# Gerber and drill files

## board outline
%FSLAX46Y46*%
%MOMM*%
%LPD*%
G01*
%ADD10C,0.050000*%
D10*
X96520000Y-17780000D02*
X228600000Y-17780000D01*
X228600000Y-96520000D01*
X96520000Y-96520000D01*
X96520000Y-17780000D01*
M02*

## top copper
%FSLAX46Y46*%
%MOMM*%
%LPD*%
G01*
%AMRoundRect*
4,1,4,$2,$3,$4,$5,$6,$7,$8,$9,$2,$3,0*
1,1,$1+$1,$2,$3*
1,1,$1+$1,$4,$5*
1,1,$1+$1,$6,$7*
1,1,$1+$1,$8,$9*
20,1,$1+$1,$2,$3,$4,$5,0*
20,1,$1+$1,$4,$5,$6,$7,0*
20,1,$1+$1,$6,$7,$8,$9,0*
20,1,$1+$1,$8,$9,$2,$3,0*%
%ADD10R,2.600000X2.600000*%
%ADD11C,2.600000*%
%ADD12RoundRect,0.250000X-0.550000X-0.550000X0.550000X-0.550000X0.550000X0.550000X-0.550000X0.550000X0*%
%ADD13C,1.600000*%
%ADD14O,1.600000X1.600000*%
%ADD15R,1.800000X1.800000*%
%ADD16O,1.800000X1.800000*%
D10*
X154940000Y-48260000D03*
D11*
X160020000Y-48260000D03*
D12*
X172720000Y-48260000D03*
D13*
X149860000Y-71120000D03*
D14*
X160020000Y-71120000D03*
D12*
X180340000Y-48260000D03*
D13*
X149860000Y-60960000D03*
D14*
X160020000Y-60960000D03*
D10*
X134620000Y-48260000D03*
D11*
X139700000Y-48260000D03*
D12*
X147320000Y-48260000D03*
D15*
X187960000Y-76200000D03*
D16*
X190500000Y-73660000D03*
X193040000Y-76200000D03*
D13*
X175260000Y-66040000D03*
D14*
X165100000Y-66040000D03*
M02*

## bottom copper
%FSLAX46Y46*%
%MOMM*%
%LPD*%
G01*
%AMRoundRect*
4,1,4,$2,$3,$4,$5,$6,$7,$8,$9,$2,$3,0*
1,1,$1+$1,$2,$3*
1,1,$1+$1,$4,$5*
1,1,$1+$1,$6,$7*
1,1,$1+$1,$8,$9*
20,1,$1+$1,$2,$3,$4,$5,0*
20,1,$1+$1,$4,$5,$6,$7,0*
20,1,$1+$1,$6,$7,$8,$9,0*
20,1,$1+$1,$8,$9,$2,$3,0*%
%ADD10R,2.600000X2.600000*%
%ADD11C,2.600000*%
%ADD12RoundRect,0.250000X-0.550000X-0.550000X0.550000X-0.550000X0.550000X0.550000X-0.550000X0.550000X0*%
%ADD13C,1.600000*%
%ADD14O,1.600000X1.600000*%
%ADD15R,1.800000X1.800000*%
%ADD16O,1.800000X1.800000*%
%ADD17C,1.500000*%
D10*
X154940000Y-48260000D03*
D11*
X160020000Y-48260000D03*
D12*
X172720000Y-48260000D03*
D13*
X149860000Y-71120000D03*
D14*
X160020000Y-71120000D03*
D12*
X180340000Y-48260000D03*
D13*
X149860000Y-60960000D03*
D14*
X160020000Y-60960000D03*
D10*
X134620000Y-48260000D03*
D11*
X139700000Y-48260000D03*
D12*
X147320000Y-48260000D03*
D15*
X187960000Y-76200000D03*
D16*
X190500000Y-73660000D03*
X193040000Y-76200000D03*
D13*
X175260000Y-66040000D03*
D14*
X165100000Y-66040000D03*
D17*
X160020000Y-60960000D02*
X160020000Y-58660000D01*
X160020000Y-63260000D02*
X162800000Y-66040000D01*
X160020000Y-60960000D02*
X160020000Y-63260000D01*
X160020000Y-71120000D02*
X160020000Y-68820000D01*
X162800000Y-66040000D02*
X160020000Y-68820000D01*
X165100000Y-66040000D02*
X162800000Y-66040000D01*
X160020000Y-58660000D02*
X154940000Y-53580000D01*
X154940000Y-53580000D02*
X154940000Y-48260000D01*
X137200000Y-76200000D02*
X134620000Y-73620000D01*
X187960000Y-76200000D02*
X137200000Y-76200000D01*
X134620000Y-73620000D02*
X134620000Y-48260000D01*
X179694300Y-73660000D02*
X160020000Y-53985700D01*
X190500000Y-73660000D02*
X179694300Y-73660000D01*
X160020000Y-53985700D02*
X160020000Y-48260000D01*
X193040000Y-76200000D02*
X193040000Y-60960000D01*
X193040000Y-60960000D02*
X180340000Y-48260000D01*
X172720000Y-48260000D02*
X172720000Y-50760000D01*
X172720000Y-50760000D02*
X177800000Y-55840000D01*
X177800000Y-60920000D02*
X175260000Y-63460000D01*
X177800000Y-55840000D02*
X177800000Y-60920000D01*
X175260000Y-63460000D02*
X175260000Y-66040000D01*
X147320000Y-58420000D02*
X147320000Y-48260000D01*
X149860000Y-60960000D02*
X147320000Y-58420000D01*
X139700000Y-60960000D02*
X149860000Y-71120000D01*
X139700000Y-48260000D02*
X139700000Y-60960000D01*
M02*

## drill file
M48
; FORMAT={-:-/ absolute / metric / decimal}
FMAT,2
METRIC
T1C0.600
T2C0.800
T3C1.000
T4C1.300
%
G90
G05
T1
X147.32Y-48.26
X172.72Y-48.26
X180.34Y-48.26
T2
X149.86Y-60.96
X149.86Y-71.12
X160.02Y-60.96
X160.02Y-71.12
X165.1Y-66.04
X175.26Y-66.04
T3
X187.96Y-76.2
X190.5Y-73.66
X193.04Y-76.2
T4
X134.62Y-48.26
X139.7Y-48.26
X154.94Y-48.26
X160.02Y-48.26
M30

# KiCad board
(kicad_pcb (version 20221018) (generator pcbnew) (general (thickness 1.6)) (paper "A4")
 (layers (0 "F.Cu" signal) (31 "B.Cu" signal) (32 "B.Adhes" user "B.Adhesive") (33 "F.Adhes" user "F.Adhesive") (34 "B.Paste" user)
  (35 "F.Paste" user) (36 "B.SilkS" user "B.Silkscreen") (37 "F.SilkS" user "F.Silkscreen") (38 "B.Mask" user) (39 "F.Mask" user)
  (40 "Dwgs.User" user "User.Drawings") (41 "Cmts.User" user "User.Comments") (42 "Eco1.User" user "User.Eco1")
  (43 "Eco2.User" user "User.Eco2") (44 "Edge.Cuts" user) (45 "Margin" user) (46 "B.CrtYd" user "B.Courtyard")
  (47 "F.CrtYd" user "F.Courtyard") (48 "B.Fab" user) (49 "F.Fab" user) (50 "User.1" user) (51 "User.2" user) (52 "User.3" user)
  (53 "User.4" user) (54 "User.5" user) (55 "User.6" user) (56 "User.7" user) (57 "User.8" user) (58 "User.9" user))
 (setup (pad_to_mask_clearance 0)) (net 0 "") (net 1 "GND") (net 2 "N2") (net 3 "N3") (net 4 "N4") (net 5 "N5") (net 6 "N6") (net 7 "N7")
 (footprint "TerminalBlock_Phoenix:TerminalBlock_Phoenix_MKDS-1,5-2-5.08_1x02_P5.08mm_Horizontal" (layer "F.Cu") (at 154.94 48.26)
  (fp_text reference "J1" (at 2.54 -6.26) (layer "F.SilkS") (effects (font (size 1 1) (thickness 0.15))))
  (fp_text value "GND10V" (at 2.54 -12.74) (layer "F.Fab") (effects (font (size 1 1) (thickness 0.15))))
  (pad "1" thru_hole rect (at 0 0) (size 2.6 2.6) (drill 1.3) (layers "*.Cu" "*.Mask") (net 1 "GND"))
  (pad "2" thru_hole circle (at 5.08 0) (size 2.6 2.6) (drill 1.3) (layers "*.Cu" "*.Mask") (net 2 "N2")))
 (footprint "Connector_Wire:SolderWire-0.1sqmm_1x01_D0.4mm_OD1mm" (layer "F.Cu") (at 172.72 48.26)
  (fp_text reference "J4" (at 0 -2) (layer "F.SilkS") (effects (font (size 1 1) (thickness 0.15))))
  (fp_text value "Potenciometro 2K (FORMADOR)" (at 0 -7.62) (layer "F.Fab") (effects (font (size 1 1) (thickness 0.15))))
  (pad "1" thru_hole roundrect (at 0 0) (size 1.6 1.6) (drill 0.6) (layers "*.Cu" "*.Mask") (roundrect_rratio 0.15625) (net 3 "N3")))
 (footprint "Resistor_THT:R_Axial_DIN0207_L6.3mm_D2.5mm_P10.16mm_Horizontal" (layer "F.Cu") (at 149.86 71.12)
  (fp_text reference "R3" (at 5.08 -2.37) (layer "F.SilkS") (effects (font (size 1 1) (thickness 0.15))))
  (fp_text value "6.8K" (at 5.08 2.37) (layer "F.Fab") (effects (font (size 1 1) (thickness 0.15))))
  (pad "1" thru_hole circle (at 0 0) (size 1.6 1.6) (drill 0.8) (layers "*.Cu" "*.Mask") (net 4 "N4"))
  (pad "2" thru_hole oval (at 10.16 0) (size 1.6 1.6) (drill 0.8) (layers "*.Cu" "*.Mask") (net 1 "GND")))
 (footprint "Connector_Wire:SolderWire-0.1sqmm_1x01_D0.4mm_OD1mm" (layer "F.Cu") (at 180.34 48.26)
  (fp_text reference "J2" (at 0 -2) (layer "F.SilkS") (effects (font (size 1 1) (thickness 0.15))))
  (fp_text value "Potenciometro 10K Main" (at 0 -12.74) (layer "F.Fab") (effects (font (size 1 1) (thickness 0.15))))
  (pad "1" thru_hole roundrect (at 0 0) (size 1.6 1.6) (drill 0.6) (layers "*.Cu" "*.Mask") (roundrect_rratio 0.15625) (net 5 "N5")))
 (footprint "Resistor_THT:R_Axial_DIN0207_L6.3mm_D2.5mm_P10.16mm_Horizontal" (layer "F.Cu") (at 149.86 60.96)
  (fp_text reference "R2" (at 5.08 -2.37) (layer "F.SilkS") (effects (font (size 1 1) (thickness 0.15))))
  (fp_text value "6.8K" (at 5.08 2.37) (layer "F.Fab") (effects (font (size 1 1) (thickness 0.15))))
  (pad "1" thru_hole circle (at 0 0) (size 1.6 1.6) (drill 0.8) (layers "*.Cu" "*.Mask") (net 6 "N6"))
  (pad "2" thru_hole oval (at 10.16 0) (size 1.6 1.6) (drill 0.8) (layers "*.Cu" "*.Mask") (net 1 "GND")))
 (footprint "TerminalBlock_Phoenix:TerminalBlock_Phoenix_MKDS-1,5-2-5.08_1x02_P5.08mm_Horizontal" (layer "F.Cu") (at 134.62 48.26)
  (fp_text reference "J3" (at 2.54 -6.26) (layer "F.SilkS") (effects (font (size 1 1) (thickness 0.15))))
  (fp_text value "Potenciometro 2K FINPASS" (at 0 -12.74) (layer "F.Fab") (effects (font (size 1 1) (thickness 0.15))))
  (pad "1" thru_hole rect (at 0 0) (size 2.6 2.6) (drill 1.3) (layers "*.Cu" "*.Mask") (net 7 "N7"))
  (pad "2" thru_hole circle (at 5.08 0) (size 2.6 2.6) (drill 1.3) (layers "*.Cu" "*.Mask") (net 4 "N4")))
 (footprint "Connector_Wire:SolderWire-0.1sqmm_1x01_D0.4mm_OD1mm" (layer "F.Cu") (at 147.32 48.26)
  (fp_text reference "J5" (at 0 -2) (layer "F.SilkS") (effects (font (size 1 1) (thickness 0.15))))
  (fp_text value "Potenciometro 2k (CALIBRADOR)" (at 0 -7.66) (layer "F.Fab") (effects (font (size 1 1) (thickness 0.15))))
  (pad "1" thru_hole roundrect (at 0 0) (size 1.6 1.6) (drill 0.6) (layers "*.Cu" "*.Mask") (roundrect_rratio 0.15625) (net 6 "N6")))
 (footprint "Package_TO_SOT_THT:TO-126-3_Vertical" (layer "F.Cu") (at 187.96 76.2)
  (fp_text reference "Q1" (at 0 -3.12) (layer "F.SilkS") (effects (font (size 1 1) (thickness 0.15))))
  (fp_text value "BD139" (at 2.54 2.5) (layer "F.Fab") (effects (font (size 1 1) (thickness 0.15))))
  (pad "1" thru_hole rect (at 0 0) (size 1.8 1.8) (drill 1) (layers "*.Cu" "*.Mask") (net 7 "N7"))
  (pad "2" thru_hole oval (at 2.54 -2.54) (size 1.8 1.8) (drill 1) (layers "*.Cu" "*.Mask") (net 2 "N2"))
  (pad "3" thru_hole oval (at 5.08 0) (size 1.8 1.8) (drill 1) (layers "*.Cu" "*.Mask") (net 5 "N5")))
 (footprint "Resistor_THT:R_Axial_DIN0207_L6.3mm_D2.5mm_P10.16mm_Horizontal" (layer "B.Cu") (at 175.26 66.04 180)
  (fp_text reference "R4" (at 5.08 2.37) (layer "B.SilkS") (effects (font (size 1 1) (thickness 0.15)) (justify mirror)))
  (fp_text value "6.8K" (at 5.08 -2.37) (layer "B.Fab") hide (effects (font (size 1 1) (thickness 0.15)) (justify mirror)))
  (pad "1" thru_hole circle (at 0 0 180) (size 1.6 1.6) (drill 0.8) (layers "*.Cu" "*.Mask") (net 3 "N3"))
  (pad "2" thru_hole oval (at 10.16 0 180) (size 1.6 1.6) (drill 0.8) (layers "*.Cu" "*.Mask") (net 1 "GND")))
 (gr_rect (start 96.52 17.78) (end 228.6 96.52) (stroke (width 0.05) (type default)) (fill none) (layer "Edge.Cuts"))
 (segment (start 160.02 60.96) (end 160.02 58.66) (width 1.5) (layer "B.Cu") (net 1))
 (segment (start 160.02 63.26) (end 162.8 66.04) (width 1.5) (layer "B.Cu") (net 1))
 (segment (start 160.02 60.96) (end 160.02 63.26) (width 1.5) (layer "B.Cu") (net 1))
 (segment (start 160.02 71.12) (end 160.02 68.82) (width 1.5) (layer "B.Cu") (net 1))
 (segment (start 162.8 66.04) (end 160.02 68.82) (width 1.5) (layer "B.Cu") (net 1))
 (segment (start 165.1 66.04) (end 162.8 66.04) (width 1.5) (layer "B.Cu") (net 1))
 (segment (start 160.02 58.66) (end 154.94 53.58) (width 1.5) (layer "B.Cu") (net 1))
 (segment (start 154.94 53.58) (end 154.94 48.26) (width 1.5) (layer "B.Cu") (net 1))
 (segment (start 137.2 76.2) (end 134.62 73.62) (width 1.5) (layer "B.Cu") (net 7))
 (segment (start 187.96 76.2) (end 137.2 76.2) (width 1.5) (layer "B.Cu") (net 7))
 (segment (start 134.62 73.62) (end 134.62 48.26) (width 1.5) (layer "B.Cu") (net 7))
 (segment (start 179.6943 73.66) (end 160.02 53.9857) (width 1.5) (layer "B.Cu") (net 2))
 (segment (start 190.5 73.66) (end 179.6943 73.66) (width 1.5) (layer "B.Cu") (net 2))
 (segment (start 160.02 53.9857) (end 160.02 48.26) (width 1.5) (layer "B.Cu") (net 2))
 (segment (start 193.04 76.2) (end 193.04 60.96) (width 1.5) (layer "B.Cu") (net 5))
 (segment (start 193.04 60.96) (end 180.34 48.26) (width 1.5) (layer "B.Cu") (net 5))
 (segment (start 172.72 48.26) (end 172.72 50.76) (width 1.5) (layer "B.Cu") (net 3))
 (segment (start 172.72 50.76) (end 177.8 55.84) (width 1.5) (layer "B.Cu") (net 3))
 (segment (start 177.8 60.92) (end 175.26 63.46) (width 1.5) (layer "B.Cu") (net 3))
 (segment (start 177.8 55.84) (end 177.8 60.92) (width 1.5) (layer "B.Cu") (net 3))
 (segment (start 175.26 63.46) (end 175.26 66.04) (width 1.5) (layer "B.Cu") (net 3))
 (segment (start 147.32 58.42) (end 147.32 48.26) (width 1.5) (layer "B.Cu") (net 6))
 (segment (start 149.86 60.96) (end 147.32 58.42) (width 1.5) (layer "B.Cu") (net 6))
 (segment (start 139.7 60.96) (end 149.86 71.12) (width 1.5) (layer "B.Cu") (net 4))
 (segment (start 139.7 48.26) (end 139.7 60.96) (width 1.5) (layer "B.Cu") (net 4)))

